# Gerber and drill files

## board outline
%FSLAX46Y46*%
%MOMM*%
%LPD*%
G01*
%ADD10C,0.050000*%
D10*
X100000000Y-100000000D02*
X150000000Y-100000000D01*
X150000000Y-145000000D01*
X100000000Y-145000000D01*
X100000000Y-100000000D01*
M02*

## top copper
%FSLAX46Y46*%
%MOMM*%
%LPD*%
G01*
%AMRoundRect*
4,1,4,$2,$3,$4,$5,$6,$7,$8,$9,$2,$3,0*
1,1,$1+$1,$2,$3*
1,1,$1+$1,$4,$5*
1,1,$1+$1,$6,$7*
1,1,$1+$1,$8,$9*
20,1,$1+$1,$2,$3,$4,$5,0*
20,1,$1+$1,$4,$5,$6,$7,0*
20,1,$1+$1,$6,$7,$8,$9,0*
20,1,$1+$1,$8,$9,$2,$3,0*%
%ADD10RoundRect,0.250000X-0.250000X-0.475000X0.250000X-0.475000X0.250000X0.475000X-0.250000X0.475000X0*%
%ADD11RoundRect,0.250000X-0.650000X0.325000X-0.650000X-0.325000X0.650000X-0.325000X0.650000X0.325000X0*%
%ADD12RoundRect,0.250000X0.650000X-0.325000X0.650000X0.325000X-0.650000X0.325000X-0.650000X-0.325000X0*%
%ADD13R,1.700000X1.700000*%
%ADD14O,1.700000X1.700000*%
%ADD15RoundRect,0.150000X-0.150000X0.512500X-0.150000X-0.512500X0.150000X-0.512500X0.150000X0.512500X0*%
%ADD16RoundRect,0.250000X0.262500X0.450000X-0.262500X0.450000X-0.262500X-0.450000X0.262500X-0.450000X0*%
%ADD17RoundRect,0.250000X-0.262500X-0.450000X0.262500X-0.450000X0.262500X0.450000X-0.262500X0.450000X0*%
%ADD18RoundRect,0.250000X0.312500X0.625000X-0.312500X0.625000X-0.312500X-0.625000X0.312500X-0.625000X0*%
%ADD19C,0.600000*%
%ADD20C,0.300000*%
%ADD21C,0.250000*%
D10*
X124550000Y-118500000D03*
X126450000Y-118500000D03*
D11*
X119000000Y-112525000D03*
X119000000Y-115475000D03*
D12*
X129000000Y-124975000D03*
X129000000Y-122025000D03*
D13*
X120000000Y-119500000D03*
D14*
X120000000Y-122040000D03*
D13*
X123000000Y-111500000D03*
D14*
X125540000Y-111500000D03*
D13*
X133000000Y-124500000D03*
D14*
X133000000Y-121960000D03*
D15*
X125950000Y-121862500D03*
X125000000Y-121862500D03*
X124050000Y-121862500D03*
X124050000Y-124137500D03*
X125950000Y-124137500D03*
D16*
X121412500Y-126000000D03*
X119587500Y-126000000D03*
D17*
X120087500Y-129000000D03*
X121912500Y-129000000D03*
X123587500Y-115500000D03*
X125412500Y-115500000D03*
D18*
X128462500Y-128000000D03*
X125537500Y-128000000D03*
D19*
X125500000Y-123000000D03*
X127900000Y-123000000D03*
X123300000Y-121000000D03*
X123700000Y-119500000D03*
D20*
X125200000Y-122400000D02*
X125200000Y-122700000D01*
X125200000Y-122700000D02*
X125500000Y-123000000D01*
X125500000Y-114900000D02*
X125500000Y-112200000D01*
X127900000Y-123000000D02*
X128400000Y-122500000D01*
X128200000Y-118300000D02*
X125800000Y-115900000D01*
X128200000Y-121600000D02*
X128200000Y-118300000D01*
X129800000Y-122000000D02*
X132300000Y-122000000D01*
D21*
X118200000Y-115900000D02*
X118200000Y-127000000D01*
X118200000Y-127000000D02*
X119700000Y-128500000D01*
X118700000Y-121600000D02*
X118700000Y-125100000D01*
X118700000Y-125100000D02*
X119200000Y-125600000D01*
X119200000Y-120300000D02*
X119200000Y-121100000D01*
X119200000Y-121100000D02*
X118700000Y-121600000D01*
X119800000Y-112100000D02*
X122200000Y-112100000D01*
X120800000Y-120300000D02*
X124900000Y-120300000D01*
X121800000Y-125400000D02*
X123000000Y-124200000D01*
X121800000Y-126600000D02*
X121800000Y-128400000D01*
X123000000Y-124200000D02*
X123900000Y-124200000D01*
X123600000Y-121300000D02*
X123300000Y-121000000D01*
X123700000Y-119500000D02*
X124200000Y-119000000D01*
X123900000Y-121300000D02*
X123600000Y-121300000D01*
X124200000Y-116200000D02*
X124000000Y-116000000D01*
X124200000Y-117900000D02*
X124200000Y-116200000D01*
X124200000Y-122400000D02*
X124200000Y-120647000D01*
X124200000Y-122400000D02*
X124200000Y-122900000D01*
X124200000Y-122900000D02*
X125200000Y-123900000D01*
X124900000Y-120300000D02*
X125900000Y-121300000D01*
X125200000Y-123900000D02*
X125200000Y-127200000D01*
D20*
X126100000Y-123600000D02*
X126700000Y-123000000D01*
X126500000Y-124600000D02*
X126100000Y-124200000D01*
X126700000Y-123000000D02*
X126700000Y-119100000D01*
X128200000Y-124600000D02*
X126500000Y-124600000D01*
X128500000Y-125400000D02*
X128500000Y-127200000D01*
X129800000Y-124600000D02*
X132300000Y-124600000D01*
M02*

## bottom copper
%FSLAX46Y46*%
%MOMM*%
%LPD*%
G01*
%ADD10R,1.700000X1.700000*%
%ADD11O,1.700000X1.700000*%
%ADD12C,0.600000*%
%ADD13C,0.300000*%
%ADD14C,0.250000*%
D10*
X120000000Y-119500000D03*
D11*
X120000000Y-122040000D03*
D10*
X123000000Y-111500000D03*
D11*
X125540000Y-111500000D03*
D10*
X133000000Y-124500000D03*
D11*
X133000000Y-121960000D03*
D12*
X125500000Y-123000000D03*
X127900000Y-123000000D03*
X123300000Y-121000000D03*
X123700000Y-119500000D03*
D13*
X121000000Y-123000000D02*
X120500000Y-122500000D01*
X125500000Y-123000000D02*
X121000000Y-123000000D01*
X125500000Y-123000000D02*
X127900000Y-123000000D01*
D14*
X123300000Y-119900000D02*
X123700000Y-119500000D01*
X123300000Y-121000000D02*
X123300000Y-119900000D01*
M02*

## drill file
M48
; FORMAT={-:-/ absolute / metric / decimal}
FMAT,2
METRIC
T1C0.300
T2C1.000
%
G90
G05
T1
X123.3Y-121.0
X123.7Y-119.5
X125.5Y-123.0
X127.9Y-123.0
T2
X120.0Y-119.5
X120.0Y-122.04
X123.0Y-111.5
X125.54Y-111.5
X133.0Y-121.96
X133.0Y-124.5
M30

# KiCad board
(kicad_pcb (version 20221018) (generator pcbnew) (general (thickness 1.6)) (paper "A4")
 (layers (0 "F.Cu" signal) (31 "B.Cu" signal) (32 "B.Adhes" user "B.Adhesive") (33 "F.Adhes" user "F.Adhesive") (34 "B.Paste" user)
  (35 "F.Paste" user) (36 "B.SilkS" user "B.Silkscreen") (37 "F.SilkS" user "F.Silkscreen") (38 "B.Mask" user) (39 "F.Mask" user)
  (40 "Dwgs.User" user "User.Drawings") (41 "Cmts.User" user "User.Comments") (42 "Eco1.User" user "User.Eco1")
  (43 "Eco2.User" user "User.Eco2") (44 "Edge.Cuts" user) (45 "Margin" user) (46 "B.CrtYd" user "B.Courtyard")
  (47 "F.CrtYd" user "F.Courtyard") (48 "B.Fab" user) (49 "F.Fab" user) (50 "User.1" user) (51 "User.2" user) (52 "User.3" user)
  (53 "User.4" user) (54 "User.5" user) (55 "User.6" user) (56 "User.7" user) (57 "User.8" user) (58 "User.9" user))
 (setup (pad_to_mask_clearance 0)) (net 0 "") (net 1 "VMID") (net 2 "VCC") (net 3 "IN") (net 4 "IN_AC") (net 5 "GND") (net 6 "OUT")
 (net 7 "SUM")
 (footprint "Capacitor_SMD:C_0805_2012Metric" (layer "F.Cu") (at 125.5 118.5)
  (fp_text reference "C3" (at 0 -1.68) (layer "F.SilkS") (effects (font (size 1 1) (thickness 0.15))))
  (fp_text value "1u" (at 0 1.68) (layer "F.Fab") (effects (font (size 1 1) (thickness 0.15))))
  (pad "1" smd roundrect (at -0.95 0) (size 1 1.45) (layers "F.Cu" "F.Paste" "F.Mask") (roundrect_rratio 0.25) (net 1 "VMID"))
  (pad "2" smd roundrect (at 0.95 0) (size 1 1.45) (layers "F.Cu" "F.Paste" "F.Mask") (roundrect_rratio 0.25) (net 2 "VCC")))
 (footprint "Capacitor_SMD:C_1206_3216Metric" (layer "F.Cu") (at 119 114 -90)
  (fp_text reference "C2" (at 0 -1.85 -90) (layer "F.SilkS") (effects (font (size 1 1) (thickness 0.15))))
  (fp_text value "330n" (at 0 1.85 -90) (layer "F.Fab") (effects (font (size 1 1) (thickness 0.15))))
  (pad "1" smd roundrect (at -1.475 0 270) (size 1.15 1.8) (layers "F.Cu" "F.Paste" "F.Mask") (roundrect_rratio 0.217391) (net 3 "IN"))
  (pad "2" smd roundrect (at 1.475 0 270) (size 1.15 1.8) (layers "F.Cu" "F.Paste" "F.Mask") (roundrect_rratio 0.217391) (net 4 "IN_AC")))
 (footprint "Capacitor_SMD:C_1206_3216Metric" (layer "F.Cu") (at 129 123.5 90)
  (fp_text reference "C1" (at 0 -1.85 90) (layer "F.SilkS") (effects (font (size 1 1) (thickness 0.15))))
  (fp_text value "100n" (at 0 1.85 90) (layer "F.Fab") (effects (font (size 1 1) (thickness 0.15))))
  (pad "1" smd roundrect (at -1.475 0 90) (size 1.15 1.8) (layers "F.Cu" "F.Paste" "F.Mask") (roundrect_rratio 0.217391) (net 2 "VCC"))
  (pad "2" smd roundrect (at 1.475 0 90) (size 1.15 1.8) (layers "F.Cu" "F.Paste" "F.Mask") (roundrect_rratio 0.217391) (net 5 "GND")))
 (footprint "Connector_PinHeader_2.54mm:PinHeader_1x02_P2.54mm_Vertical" (layer "F.Cu") (at 120 119.5)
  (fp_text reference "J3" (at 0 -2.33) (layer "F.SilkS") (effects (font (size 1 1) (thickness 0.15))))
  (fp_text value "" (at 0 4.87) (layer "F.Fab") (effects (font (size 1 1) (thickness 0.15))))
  (pad "1" thru_hole rect (at 0 0) (size 1.7 1.7) (drill 1) (layers "*.Cu" "*.Mask") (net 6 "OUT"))
  (pad "2" thru_hole oval (at 0 2.54) (size 1.7 1.7) (drill 1) (layers "*.Cu" "*.Mask") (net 5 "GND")))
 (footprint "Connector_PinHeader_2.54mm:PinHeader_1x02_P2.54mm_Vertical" (layer "F.Cu") (at 123 111.5 90)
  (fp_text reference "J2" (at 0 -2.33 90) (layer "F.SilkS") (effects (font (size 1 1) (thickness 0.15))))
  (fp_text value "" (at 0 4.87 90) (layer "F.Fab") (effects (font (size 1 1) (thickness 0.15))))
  (pad "1" thru_hole rect (at 0 0 90) (size 1.7 1.7) (drill 1) (layers "*.Cu" "*.Mask") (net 3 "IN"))
  (pad "2" thru_hole oval (at 0 2.54 90) (size 1.7 1.7) (drill 1) (layers "*.Cu" "*.Mask") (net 5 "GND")))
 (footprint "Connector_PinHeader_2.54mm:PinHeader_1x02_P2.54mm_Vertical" (layer "F.Cu") (at 133 124.5 180)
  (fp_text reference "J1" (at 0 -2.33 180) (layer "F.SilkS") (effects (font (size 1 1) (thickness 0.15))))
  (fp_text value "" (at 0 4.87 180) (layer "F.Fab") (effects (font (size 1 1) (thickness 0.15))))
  (pad "1" thru_hole rect (at 0 0 180) (size 1.7 1.7) (drill 1) (layers "*.Cu" "*.Mask") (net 2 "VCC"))
  (pad "2" thru_hole oval (at 0 2.54 180) (size 1.7 1.7) (drill 1) (layers "*.Cu" "*.Mask") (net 5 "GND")))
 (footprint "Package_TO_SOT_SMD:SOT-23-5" (layer "F.Cu") (at 125 123 -90)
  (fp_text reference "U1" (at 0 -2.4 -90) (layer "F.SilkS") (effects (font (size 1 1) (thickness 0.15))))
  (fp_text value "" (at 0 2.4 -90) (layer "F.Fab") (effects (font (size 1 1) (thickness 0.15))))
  (pad "1" smd roundrect (at -1.1375 -0.95 270) (size 1.325 0.6) (layers "F.Cu" "F.Paste" "F.Mask") (roundrect_rratio 0.25) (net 6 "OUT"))
  (pad "2" smd roundrect (at -1.1375 0 270) (size 1.325 0.6) (layers "F.Cu" "F.Paste" "F.Mask") (roundrect_rratio 0.25) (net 5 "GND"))
  (pad "3" smd roundrect (at -1.1375 0.95 270) (size 1.325 0.6) (layers "F.Cu" "F.Paste" "F.Mask") (roundrect_rratio 0.25) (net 1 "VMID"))
  (pad "4" smd roundrect (at 1.1375 0.95 270) (size 1.325 0.6) (layers "F.Cu" "F.Paste" "F.Mask") (roundrect_rratio 0.25) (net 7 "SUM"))
  (pad "5" smd roundrect (at 1.1375 -0.95 270) (size 1.325 0.6) (layers "F.Cu" "F.Paste" "F.Mask") (roundrect_rratio 0.25) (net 2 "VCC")))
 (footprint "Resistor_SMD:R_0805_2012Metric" (layer "F.Cu") (at 120.5 126 180)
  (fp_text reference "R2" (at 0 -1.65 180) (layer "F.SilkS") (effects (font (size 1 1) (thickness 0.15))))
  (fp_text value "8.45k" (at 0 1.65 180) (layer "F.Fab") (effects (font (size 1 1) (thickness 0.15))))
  (pad "1" smd roundrect (at -0.9125 0 180) (size 1.025 1.4) (layers "F.Cu" "F.Paste" "F.Mask") (roundrect_rratio 0.243902) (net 7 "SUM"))
  (pad "2" smd roundrect (at 0.9125 0 180) (size 1.025 1.4) (layers "F.Cu" "F.Paste" "F.Mask") (roundrect_rratio 0.243902) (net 6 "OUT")))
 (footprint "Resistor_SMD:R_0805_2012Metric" (layer "F.Cu") (at 121 129)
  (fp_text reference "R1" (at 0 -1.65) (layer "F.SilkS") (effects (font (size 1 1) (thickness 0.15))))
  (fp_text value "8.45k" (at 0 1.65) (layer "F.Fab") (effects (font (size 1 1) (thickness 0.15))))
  (pad "1" smd roundrect (at -0.9125 0) (size 1.025 1.4) (layers "F.Cu" "F.Paste" "F.Mask") (roundrect_rratio 0.243902) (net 4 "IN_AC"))
  (pad "2" smd roundrect (at 0.9125 0) (size 1.025 1.4) (layers "F.Cu" "F.Paste" "F.Mask") (roundrect_rratio 0.243902) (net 7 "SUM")))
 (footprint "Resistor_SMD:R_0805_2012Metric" (layer "F.Cu") (at 124.5 115.5)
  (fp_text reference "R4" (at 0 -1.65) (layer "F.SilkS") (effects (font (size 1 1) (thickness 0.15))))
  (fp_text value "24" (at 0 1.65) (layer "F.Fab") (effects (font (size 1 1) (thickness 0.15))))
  (pad "1" smd roundrect (at -0.9125 0) (size 1.025 1.4) (layers "F.Cu" "F.Paste" "F.Mask") (roundrect_rratio 0.243902) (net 1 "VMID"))
  (pad "2" smd roundrect (at 0.9125 0) (size 1.025 1.4) (layers "F.Cu" "F.Paste" "F.Mask") (roundrect_rratio 0.243902) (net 5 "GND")))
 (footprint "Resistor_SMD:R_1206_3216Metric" (layer "F.Cu") (at 127 128 180)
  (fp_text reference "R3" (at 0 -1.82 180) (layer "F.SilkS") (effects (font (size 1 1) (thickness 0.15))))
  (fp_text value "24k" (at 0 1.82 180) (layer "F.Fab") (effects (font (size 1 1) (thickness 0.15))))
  (pad "1" smd roundrect (at -1.4625 0 180) (size 1.125 1.75) (layers "F.Cu" "F.Paste" "F.Mask") (roundrect_rratio 0.222222) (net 2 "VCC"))
  (pad "2" smd roundrect (at 1.4625 0 180) (size 1.125 1.75) (layers "F.Cu" "F.Paste" "F.Mask") (roundrect_rratio 0.222222) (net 1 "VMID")))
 (gr_rect (start 100 100) (end 150 145) (stroke (width 0.05) (type default)) (fill none) (layer "Edge.Cuts"))
 (segment (start 125.2 122.4) (end 125.2 122.7) (width 0.3) (layer "F.Cu") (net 5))
 (segment (start 125.2 122.7) (end 125.5 123) (width 0.3) (layer "F.Cu") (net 5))
 (segment (start 125.5 114.9) (end 125.5 112.2) (width 0.3) (layer "F.Cu") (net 5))
 (segment (start 127.9 123) (end 128.4 122.5) (width 0.3) (layer "F.Cu") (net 5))
 (segment (start 128.2 118.3) (end 125.8 115.9) (width 0.3) (layer "F.Cu") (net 5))
 (segment (start 128.2 121.6) (end 128.2 118.3) (width 0.3) (layer "F.Cu") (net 5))
 (segment (start 129.8 122) (end 132.3 122) (width 0.3) (layer "F.Cu") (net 5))
 (via (at 125.5 123) (size 0.6) (drill 0.3) (layers "F.Cu" "B.Cu") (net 5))
 (via (at 127.9 123) (size 0.6) (drill 0.3) (layers "F.Cu" "B.Cu") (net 5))
 (segment (start 118.2 115.9) (end 118.2 127) (width 0.25) (layer "F.Cu") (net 4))
 (segment (start 118.2 127) (end 119.7 128.5) (width 0.25) (layer "F.Cu") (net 4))
 (segment (start 118.7 121.6) (end 118.7 125.1) (width 0.25) (layer "F.Cu") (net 6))
 (segment (start 118.7 125.1) (end 119.2 125.6) (width 0.25) (layer "F.Cu") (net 6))
 (segment (start 119.2 120.3) (end 119.2 121.1) (width 0.25) (layer "F.Cu") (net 6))
 (segment (start 119.2 121.1) (end 118.7 121.6) (width 0.25) (layer "F.Cu") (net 6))
 (segment (start 119.8 112.1) (end 122.2 112.1) (width 0.25) (layer "F.Cu") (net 3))
 (segment (start 120.8 120.3) (end 124.9 120.3) (width 0.25) (layer "F.Cu") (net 6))
 (segment (start 121 123) (end 120.5 122.5) (width 0.3) (layer "B.Cu") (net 5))
 (segment (start 121.8 125.4) (end 123 124.2) (width 0.25) (layer "F.Cu") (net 7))
 (segment (start 121.8 126.6) (end 121.8 128.4) (width 0.25) (layer "F.Cu") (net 7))
 (segment (start 123 124.2) (end 123.9 124.2) (width 0.25) (layer "F.Cu") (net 7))
 (segment (start 123.6 121.3) (end 123.3 121) (width 0.25) (layer "F.Cu") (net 1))
 (segment (start 123.7 119.5) (end 124.2 119) (width 0.25) (layer "F.Cu") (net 1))
 (segment (start 123.9 121.3) (end 123.6 121.3) (width 0.25) (layer "F.Cu") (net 1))
 (segment (start 124.2 116.2) (end 124 116) (width 0.25) (layer "F.Cu") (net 1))
 (segment (start 124.2 117.9) (end 124.2 116.2) (width 0.25) (layer "F.Cu") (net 1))
 (segment (start 124.2 122.4) (end 124.2 120.647) (width 0.25) (layer "F.Cu") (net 1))
 (segment (start 124.2 122.4) (end 124.2 122.9) (width 0.25) (layer "F.Cu") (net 1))
 (segment (start 124.2 122.9) (end 125.2 123.9) (width 0.25) (layer "F.Cu") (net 1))
 (segment (start 124.9 120.3) (end 125.9 121.3) (width 0.25) (layer "F.Cu") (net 6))
 (segment (start 125.2 123.9) (end 125.2 127.2) (width 0.25) (layer "F.Cu") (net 1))
 (segment (start 125.5 123) (end 121 123) (width 0.3) (layer "B.Cu") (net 5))
 (segment (start 125.5 123) (end 127.9 123) (width 0.3) (layer "B.Cu") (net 5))
 (segment (start 126.1 123.6) (end 126.7 123) (width 0.3) (layer "F.Cu") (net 2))
 (segment (start 126.5 124.6) (end 126.1 124.2) (width 0.3) (layer "F.Cu") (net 2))
 (segment (start 126.7 123) (end 126.7 119.1) (width 0.3) (layer "F.Cu") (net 2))
 (segment (start 128.2 124.6) (end 126.5 124.6) (width 0.3) (layer "F.Cu") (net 2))
 (segment (start 128.5 125.4) (end 128.5 127.2) (width 0.3) (layer "F.Cu") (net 2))
 (segment (start 129.8 124.6) (end 132.3 124.6) (width 0.3) (layer "F.Cu") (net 2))
 (via (at 123.3 121) (size 0.6) (drill 0.3) (layers "F.Cu" "B.Cu") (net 1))
 (via (at 123.7 119.5) (size 0.6) (drill 0.3) (layers "F.Cu" "B.Cu") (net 1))
 (segment (start 123.3 119.9) (end 123.7 119.5) (width 0.25) (layer "B.Cu") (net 1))
 (segment (start 123.3 121) (end 123.3 119.9) (width 0.25) (layer "B.Cu") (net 1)))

